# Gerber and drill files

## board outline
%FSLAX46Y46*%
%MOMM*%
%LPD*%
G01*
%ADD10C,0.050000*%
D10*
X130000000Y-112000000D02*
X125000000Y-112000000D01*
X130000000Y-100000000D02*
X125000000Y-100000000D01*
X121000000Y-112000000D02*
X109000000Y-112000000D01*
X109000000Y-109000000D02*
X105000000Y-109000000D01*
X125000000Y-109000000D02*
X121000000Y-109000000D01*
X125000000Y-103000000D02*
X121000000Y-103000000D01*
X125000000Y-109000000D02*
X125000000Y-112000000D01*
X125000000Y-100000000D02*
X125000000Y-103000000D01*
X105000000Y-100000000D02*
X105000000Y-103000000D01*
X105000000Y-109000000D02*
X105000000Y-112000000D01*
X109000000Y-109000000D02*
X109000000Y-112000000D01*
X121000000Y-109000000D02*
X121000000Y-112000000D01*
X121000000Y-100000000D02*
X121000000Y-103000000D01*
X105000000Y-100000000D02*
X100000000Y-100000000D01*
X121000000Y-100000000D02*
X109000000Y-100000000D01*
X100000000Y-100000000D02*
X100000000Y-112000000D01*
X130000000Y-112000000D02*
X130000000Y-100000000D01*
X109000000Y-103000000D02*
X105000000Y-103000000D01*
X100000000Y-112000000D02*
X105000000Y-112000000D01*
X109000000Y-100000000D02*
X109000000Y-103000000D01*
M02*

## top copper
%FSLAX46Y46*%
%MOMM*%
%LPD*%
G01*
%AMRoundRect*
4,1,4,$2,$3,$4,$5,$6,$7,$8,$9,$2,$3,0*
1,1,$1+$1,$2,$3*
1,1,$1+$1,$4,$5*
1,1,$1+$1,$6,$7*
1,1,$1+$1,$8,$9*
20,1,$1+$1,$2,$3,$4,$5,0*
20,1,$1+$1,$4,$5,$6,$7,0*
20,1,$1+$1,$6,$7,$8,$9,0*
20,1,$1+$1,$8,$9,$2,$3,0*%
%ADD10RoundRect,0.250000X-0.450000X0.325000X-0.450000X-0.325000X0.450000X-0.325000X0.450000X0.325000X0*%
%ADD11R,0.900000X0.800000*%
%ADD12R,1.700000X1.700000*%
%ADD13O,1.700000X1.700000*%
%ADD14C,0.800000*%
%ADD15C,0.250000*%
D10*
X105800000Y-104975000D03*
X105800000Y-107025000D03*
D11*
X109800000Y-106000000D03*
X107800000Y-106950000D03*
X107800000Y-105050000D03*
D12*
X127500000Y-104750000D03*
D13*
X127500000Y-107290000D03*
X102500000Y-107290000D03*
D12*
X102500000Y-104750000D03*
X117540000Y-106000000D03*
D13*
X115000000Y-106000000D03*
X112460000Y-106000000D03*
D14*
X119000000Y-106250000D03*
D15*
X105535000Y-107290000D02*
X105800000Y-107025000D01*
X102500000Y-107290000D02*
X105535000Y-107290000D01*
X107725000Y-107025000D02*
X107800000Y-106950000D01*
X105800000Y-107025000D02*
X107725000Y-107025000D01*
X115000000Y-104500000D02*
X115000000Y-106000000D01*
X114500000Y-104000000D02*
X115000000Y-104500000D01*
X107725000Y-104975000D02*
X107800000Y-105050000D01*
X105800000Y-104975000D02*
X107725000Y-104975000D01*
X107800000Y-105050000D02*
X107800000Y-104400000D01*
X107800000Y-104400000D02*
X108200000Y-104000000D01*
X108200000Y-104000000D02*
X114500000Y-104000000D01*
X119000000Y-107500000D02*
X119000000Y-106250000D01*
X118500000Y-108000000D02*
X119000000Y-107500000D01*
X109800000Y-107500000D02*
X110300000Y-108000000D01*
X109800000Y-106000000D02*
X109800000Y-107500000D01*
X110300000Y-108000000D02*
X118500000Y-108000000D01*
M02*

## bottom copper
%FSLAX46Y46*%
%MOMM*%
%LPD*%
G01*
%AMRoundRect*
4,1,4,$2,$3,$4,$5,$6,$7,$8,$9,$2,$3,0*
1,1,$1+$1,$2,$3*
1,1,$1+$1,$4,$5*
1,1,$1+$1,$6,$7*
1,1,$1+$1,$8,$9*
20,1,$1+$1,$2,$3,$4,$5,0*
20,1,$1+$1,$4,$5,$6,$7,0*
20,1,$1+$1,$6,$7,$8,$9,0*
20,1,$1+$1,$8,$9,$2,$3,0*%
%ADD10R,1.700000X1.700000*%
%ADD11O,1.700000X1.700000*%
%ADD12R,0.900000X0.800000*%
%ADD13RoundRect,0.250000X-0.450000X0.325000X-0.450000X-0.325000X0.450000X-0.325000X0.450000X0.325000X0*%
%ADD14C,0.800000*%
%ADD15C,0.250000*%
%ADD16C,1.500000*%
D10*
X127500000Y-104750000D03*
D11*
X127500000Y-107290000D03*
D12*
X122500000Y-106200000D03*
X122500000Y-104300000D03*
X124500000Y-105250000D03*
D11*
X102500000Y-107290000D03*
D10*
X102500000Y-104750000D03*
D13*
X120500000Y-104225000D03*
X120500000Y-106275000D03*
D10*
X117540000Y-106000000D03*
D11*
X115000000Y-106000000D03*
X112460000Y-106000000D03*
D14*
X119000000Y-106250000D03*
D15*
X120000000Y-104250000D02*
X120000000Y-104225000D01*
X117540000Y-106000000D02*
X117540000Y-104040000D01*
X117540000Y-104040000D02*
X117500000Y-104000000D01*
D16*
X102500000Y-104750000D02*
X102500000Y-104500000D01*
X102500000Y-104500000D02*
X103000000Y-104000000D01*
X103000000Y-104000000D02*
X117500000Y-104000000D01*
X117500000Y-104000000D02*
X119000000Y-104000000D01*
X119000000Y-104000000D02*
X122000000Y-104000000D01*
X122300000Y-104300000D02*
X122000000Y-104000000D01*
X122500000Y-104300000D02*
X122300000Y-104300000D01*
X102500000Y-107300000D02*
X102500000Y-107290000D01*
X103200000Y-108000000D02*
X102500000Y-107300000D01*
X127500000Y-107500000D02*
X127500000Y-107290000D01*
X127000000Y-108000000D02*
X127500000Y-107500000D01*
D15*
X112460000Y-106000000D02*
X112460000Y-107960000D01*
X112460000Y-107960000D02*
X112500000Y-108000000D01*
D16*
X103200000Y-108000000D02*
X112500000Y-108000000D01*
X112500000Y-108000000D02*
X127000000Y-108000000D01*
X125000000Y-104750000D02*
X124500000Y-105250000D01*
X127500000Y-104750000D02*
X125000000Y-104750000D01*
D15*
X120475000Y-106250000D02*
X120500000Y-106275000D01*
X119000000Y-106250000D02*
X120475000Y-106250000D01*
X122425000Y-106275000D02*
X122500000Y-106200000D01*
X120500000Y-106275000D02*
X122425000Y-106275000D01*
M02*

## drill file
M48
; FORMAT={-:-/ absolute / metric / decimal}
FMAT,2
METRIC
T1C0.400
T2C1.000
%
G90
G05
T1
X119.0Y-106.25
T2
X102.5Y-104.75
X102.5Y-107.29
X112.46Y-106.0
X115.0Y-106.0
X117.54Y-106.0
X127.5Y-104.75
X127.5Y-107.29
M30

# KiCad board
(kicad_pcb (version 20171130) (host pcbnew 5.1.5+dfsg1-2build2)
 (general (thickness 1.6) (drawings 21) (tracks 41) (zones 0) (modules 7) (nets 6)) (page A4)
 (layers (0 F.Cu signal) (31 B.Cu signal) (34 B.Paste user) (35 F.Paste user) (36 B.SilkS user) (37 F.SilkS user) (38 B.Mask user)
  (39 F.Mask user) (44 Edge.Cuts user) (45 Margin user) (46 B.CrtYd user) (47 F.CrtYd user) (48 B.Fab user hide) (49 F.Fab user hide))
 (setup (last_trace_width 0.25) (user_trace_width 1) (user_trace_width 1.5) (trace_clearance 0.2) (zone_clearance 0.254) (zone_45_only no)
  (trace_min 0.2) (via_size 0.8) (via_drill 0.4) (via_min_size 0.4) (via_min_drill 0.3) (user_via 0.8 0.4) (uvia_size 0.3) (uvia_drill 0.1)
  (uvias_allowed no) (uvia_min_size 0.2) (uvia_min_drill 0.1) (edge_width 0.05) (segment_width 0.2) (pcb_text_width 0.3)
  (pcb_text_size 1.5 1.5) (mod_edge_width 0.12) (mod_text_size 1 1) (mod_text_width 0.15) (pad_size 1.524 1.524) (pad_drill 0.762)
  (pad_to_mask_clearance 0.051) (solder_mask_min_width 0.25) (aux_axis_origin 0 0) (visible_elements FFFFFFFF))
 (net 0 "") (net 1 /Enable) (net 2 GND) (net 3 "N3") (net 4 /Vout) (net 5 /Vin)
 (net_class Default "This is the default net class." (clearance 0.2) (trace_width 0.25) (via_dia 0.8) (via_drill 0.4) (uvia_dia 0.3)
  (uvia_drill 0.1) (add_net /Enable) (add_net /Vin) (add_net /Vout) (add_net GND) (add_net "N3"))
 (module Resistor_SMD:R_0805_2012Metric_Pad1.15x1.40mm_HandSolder (layer F.Cu) (at 105.8 106 270)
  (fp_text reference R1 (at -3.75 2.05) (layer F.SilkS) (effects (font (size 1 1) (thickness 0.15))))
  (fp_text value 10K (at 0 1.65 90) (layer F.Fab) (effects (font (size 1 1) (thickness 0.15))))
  (pad 1 smd roundrect (at -1.025 0 270) (size 1.15 1.4) (layers F.Cu F.Paste F.Mask) (roundrect_rratio 0.217391) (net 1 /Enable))
  (pad 2 smd roundrect (at 1.025 0 270) (size 1.15 1.4) (layers F.Cu F.Paste F.Mask) (roundrect_rratio 0.217391) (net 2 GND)))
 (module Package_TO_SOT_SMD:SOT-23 (layer F.Cu) (at 108.8 106)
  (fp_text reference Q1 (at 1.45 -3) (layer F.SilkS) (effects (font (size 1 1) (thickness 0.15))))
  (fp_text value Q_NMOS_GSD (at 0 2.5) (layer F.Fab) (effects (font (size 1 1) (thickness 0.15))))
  (pad 3 smd rect (at 1 0) (size 0.9 0.8) (layers F.Cu F.Paste F.Mask) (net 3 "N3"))
  (pad 2 smd rect (at -1 0.95) (size 0.9 0.8) (layers F.Cu F.Paste F.Mask) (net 2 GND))
  (pad 1 smd rect (at -1 -0.95) (size 0.9 0.8) (layers F.Cu F.Paste F.Mask) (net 1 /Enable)))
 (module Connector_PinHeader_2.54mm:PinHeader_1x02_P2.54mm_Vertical (layer F.Cu) (at 127.5 104.75)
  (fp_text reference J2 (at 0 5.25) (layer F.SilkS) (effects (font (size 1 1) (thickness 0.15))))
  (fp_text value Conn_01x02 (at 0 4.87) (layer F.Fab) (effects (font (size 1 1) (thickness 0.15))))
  (pad 1 thru_hole rect (at 0 0) (size 1.7 1.7) (drill 1) (layers *.Cu *.Mask) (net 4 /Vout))
  (pad 2 thru_hole oval (at 0 2.54) (size 1.7 1.7) (drill 1) (layers *.Cu *.Mask) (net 2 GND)))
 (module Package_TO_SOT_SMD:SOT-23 (layer B.Cu) (at 123.5 105.25)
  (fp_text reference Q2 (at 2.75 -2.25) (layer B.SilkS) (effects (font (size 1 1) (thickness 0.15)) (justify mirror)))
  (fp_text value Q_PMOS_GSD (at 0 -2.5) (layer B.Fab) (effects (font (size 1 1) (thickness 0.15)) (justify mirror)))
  (pad 1 smd rect (at -1 0.95) (size 0.9 0.8) (layers B.Cu B.Paste B.Mask) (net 3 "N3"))
  (pad 2 smd rect (at -1 -0.95) (size 0.9 0.8) (layers B.Cu B.Paste B.Mask) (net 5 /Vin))
  (pad 3 smd rect (at 1 0) (size 0.9 0.8) (layers B.Cu B.Paste B.Mask) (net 4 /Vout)))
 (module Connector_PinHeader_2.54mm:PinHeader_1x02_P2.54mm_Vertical (layer F.Cu) (at 102.5 104.75)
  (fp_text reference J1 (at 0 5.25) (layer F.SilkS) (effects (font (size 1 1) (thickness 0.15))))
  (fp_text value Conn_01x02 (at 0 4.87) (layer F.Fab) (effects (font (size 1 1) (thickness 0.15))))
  (pad 2 thru_hole oval (at 0 2.54) (size 1.7 1.7) (drill 1) (layers *.Cu *.Mask) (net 2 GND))
  (pad 1 thru_hole rect (at 0 0) (size 1.7 1.7) (drill 1) (layers *.Cu *.Mask) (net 5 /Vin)))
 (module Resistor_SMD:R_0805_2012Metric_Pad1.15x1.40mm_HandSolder (layer B.Cu) (at 120.5 105.25 270)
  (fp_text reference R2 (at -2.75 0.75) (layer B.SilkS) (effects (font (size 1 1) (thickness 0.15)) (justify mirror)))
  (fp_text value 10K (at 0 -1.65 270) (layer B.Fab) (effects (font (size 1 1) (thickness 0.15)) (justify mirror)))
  (pad 1 smd roundrect (at -1.025 0 270) (size 1.15 1.4) (layers B.Cu B.Paste B.Mask) (roundrect_rratio 0.217391) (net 5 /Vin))
  (pad 2 smd roundrect (at 1.025 0 270) (size 1.15 1.4) (layers B.Cu B.Paste B.Mask) (roundrect_rratio 0.217391) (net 3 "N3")))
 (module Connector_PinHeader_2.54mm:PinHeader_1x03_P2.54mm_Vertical (layer F.Cu) (at 117.54 106 270)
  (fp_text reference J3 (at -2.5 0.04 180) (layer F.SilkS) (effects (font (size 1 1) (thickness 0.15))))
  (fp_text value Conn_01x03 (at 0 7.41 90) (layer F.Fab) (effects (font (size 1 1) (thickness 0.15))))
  (pad 1 thru_hole rect (at 0 0 270) (size 1.7 1.7) (drill 1) (layers *.Cu *.Mask) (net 5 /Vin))
  (pad 2 thru_hole oval (at 0 2.54 270) (size 1.7 1.7) (drill 1) (layers *.Cu *.Mask) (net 1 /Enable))
  (pad 3 thru_hole oval (at 0 5.08 270) (size 1.7 1.7) (drill 1) (layers *.Cu *.Mask) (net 2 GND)))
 (gr_line (start 130 112) (end 125 112) (layer Edge.Cuts) (width 0.05))
 (gr_line (start 130 100) (end 125 100) (layer Edge.Cuts) (width 0.05))
 (gr_line (start 121 112) (end 109 112) (layer Edge.Cuts) (width 0.05))
 (gr_line (start 109 109) (end 105 109) (layer Edge.Cuts) (width 0.05))
 (gr_line (start 125 109) (end 121 109) (layer Edge.Cuts) (width 0.05))
 (gr_line (start 125 103) (end 121 103) (layer Edge.Cuts) (width 0.05))
 (gr_line (start 125 109) (end 125 112) (layer Edge.Cuts) (width 0.05))
 (gr_line (start 125 100) (end 125 103) (layer Edge.Cuts) (width 0.05))
 (gr_line (start 105 100) (end 105 103) (layer Edge.Cuts) (width 0.05))
 (gr_line (start 105 109) (end 105 112) (layer Edge.Cuts) (width 0.05))
 (gr_line (start 109 109) (end 109 112) (layer Edge.Cuts) (width 0.05))
 (gr_line (start 121 109) (end 121 112) (layer Edge.Cuts) (width 0.05))
 (gr_line (start 121 100) (end 121 103) (layer Edge.Cuts) (width 0.05))
 (gr_line (start 105 100) (end 100 100) (layer Edge.Cuts) (width 0.05))
 (gr_line (start 121 100) (end 109 100) (layer Edge.Cuts) (width 0.05))
 (gr_line (start 100 100) (end 100 112) (layer Edge.Cuts) (width 0.05))
 (gr_line (start 130 112) (end 130 100) (layer Edge.Cuts) (width 0.05))
 (gr_line (start 109 103) (end 105 103) (layer Edge.Cuts) (width 0.05))
 (gr_line (start 100 112) (end 105 112) (layer Edge.Cuts) (width 0.05))
 (gr_line (start 109 100) (end 109 103) (layer Edge.Cuts) (width 0.05))
 (segment (start 120 104.25) (end 120 104.225) (width 0.25) (layer B.Cu) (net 5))
 (segment (start 117.54 106) (end 117.54 104.04) (width 0.25) (layer B.Cu) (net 5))
 (segment (start 117.54 104.04) (end 117.5 104) (width 0.25) (layer B.Cu) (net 5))
 (segment (start 102.5 104.75) (end 102.5 104.5) (width 1.5) (layer B.Cu) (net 5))
 (segment (start 102.5 104.5) (end 103 104) (width 1.5) (layer B.Cu) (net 5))
 (segment (start 103 104) (end 117.5 104) (width 1.5) (layer B.Cu) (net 5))
 (segment (start 117.5 104) (end 119 104) (width 1.5) (layer B.Cu) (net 5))
 (segment (start 119 104) (end 122 104) (width 1.5) (layer B.Cu) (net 5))
 (segment (start 122.3 104.3) (end 122 104) (width 1.5) (layer B.Cu) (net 5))
 (segment (start 122.5 104.3) (end 122.3 104.3) (width 1.5) (layer B.Cu) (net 5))
 (segment (start 102.5 107.3) (end 102.5 107.29) (width 1.5) (layer B.Cu) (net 2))
 (segment (start 103.2 108) (end 102.5 107.3) (width 1.5) (layer B.Cu) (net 2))
 (segment (start 105.535 107.29) (end 105.8 107.025) (width 0.25) (layer F.Cu) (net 2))
 (segment (start 102.5 107.29) (end 105.535 107.29) (width 0.25) (layer F.Cu) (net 2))
 (segment (start 107.725 107.025) (end 107.8 106.95) (width 0.25) (layer F.Cu) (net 2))
 (segment (start 105.8 107.025) (end 107.725 107.025) (width 0.25) (layer F.Cu) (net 2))
 (segment (start 127.5 107.5) (end 127.5 107.29) (width 1.5) (layer B.Cu) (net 2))
 (segment (start 127 108) (end 127.5 107.5) (width 1.5) (layer B.Cu) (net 2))
 (segment (start 112.46 106) (end 112.46 107.96) (width 0.25) (layer B.Cu) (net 2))
 (segment (start 112.46 107.96) (end 112.5 108) (width 0.25) (layer B.Cu) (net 2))
 (segment (start 103.2 108) (end 112.5 108) (width 1.5) (layer B.Cu) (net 2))
 (segment (start 112.5 108) (end 127 108) (width 1.5) (layer B.Cu) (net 2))
 (segment (start 125 104.75) (end 124.5 105.25) (width 1.5) (layer B.Cu) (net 4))
 (segment (start 127.5 104.75) (end 125 104.75) (width 1.5) (layer B.Cu) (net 4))
 (segment (start 115 104.5) (end 115 106) (width 0.25) (layer F.Cu) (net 1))
 (segment (start 114.5 104) (end 115 104.5) (width 0.25) (layer F.Cu) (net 1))
 (segment (start 107.725 104.975) (end 107.8 105.05) (width 0.25) (layer F.Cu) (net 1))
 (segment (start 105.8 104.975) (end 107.725 104.975) (width 0.25) (layer F.Cu) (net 1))
 (segment (start 107.8 105.05) (end 107.8 104.4) (width 0.25) (layer F.Cu) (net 1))
 (segment (start 107.8 104.4) (end 108.2 104) (width 0.25) (layer F.Cu) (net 1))
 (segment (start 108.2 104) (end 114.5 104) (width 0.25) (layer F.Cu) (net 1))
 (via (at 119 106.25) (size 0.8) (drill 0.4) (layers F.Cu B.Cu) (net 3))
 (segment (start 119 107.5) (end 119 106.25) (width 0.25) (layer F.Cu) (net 3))
 (segment (start 118.5 108) (end 119 107.5) (width 0.25) (layer F.Cu) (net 3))
 (segment (start 120.475 106.25) (end 120.5 106.275) (width 0.25) (layer B.Cu) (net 3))
 (segment (start 119 106.25) (end 120.475 106.25) (width 0.25) (layer B.Cu) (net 3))
 (segment (start 122.425 106.275) (end 122.5 106.2) (width 0.25) (layer B.Cu) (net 3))
 (segment (start 120.5 106.275) (end 122.425 106.275) (width 0.25) (layer B.Cu) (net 3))
 (segment (start 109.8 107.5) (end 110.3 108) (width 0.25) (layer F.Cu) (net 3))
 (segment (start 109.8 106) (end 109.8 107.5) (width 0.25) (layer F.Cu) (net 3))
 (segment (start 110.3 108) (end 118.5 108) (width 0.25) (layer F.Cu) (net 3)))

